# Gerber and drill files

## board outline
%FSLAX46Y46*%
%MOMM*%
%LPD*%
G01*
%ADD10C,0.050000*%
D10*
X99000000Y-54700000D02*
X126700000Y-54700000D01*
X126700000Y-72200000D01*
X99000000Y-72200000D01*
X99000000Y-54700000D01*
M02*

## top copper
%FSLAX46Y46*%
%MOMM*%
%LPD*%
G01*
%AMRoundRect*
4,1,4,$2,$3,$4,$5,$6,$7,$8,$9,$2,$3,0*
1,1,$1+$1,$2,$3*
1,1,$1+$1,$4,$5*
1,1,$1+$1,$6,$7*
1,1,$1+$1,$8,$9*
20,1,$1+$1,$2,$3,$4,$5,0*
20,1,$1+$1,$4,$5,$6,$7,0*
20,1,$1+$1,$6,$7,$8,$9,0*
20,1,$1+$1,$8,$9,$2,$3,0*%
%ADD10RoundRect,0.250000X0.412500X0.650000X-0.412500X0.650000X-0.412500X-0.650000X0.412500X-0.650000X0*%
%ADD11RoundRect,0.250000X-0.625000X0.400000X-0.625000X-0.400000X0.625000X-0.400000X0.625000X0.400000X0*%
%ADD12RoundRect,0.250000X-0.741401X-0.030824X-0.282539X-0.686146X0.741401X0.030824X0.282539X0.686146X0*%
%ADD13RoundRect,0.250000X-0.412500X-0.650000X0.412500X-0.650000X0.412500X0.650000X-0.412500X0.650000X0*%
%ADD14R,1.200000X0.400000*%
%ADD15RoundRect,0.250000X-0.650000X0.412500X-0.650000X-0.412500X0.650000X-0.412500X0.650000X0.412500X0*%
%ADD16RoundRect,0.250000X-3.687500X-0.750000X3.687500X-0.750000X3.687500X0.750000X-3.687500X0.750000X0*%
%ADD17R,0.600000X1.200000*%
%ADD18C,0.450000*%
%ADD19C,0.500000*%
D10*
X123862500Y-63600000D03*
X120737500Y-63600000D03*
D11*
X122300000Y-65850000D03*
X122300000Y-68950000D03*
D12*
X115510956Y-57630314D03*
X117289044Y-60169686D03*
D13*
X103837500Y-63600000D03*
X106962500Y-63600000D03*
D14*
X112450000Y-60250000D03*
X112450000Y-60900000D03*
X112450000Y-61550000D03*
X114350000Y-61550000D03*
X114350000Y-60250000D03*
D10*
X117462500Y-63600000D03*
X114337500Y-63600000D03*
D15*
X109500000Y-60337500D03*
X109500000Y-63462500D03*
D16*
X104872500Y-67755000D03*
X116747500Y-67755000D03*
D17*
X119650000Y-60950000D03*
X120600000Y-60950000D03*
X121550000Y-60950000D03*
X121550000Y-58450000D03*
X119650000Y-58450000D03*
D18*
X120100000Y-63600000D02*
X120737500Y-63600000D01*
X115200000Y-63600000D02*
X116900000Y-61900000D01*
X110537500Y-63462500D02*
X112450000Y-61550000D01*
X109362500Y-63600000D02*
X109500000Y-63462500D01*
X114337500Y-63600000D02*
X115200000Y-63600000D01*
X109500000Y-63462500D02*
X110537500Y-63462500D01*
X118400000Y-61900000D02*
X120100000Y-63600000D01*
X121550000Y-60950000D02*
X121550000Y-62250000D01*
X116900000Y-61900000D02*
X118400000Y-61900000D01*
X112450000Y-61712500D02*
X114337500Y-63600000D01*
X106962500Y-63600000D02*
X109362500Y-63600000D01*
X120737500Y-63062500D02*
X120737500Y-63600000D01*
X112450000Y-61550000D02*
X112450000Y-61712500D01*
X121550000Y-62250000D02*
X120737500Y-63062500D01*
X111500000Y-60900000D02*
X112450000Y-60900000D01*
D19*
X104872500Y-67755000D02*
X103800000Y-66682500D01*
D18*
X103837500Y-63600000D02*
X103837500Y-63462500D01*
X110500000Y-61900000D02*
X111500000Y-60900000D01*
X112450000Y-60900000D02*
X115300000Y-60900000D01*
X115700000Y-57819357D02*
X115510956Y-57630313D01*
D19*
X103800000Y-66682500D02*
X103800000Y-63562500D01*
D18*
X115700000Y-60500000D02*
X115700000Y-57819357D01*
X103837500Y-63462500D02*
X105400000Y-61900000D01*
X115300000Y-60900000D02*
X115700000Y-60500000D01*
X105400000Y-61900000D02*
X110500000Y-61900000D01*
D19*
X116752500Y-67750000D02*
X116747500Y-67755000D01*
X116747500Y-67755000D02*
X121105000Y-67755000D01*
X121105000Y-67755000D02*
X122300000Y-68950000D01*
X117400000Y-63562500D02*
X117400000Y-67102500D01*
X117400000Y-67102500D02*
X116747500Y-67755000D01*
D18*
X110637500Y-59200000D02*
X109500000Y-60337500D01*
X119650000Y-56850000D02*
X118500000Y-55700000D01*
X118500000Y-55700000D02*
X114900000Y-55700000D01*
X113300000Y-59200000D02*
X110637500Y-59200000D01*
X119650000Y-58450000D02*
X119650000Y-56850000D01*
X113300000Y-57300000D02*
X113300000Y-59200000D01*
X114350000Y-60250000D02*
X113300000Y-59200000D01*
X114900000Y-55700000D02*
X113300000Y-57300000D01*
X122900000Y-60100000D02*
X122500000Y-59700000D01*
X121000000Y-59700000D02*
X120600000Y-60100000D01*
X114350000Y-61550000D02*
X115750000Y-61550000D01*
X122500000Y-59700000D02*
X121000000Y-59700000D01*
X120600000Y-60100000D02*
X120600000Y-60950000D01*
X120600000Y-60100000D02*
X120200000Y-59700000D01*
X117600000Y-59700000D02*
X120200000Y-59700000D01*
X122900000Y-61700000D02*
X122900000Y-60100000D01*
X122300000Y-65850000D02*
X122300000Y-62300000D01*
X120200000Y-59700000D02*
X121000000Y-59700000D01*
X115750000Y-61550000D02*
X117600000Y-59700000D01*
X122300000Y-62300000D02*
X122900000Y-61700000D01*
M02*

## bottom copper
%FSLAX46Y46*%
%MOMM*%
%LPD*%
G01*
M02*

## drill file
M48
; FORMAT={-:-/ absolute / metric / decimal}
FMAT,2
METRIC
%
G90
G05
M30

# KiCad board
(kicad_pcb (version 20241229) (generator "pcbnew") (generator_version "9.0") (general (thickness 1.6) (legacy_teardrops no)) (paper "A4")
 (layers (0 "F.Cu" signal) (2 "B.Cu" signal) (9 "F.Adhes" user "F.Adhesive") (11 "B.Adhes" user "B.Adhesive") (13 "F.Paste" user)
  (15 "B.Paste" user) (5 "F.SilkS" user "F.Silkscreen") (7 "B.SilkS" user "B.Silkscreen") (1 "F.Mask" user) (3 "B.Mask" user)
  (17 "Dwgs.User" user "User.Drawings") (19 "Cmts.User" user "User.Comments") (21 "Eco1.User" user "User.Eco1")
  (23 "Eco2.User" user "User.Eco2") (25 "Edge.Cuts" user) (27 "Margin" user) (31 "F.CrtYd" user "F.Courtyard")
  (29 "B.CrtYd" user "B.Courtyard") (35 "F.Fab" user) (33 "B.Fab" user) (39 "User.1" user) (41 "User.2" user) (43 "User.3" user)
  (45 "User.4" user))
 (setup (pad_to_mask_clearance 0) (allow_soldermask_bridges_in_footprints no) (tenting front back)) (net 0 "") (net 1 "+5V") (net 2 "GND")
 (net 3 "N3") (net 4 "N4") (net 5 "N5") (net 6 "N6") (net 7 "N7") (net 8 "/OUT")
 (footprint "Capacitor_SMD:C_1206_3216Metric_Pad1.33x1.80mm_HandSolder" (layer "F.Cu") (at 122.3 63.6 180)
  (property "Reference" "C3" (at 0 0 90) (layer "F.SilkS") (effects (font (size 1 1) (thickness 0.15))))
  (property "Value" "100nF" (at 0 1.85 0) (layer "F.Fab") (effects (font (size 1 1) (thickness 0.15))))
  (pad "1" smd roundrect (at -1.5625 0 180) (size 1.325 1.8) (layers "F.Cu" "F.Mask" "F.Paste") (roundrect_rratio 0.188679) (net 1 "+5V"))
  (pad "2" smd roundrect (at 1.5625 0 180) (size 1.325 1.8) (layers "F.Cu" "F.Mask" "F.Paste") (roundrect_rratio 0.188679) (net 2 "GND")))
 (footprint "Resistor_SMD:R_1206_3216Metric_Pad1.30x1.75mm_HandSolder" (layer "F.Cu") (at 122.3 67.4 -90)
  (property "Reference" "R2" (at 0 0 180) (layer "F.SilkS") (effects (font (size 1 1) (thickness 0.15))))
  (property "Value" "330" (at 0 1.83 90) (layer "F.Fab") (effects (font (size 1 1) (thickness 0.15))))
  (pad "1" smd roundrect (at -1.55 0 270) (size 1.3 1.75) (layers "F.Cu" "F.Mask" "F.Paste") (roundrect_rratio 0.192308) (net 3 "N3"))
  (pad "2" smd roundrect (at 1.55 0 270) (size 1.3 1.75) (layers "F.Cu" "F.Mask" "F.Paste") (roundrect_rratio 0.192308) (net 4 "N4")))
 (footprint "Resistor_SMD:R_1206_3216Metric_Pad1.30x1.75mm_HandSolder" (layer "F.Cu") (at 116.4 58.9 -55)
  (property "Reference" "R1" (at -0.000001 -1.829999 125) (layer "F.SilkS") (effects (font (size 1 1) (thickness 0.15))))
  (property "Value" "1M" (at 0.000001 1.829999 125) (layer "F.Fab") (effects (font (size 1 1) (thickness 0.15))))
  (pad "1" smd roundrect (at -1.550001 0 305) (size 1.3 1.75) (layers "F.Cu" "F.Mask" "F.Paste") (roundrect_rratio 0.192308) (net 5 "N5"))
  (pad "2" smd roundrect (at 1.550001 0 305) (size 1.3 1.75) (layers "F.Cu" "F.Mask" "F.Paste") (roundrect_rratio 0.192308) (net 3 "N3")))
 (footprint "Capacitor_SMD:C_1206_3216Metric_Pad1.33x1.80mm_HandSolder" (layer "F.Cu") (at 105.4 63.6)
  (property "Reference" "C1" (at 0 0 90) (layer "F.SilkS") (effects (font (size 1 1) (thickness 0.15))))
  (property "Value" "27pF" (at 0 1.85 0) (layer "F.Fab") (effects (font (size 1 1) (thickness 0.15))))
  (pad "1" smd roundrect (at -1.5625 0) (size 1.325 1.8) (layers "F.Cu" "F.Mask" "F.Paste") (roundrect_rratio 0.188679) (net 5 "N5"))
  (pad "2" smd roundrect (at 1.5625 0) (size 1.325 1.8) (layers "F.Cu" "F.Mask" "F.Paste") (roundrect_rratio 0.188679) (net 2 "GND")))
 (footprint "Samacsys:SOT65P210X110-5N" (layer "F.Cu") (at 113.4 60.9)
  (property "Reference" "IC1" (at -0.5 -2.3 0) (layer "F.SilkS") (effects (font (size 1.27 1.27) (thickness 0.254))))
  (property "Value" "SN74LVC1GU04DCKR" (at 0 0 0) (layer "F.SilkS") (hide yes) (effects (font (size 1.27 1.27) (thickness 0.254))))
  (pad "1" smd rect (at -0.95 -0.65 90) (size 0.4 1.2) (layers "F.Cu" "F.Mask" "F.Paste") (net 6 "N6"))
  (pad "2" smd rect (at -0.95 0 90) (size 0.4 1.2) (layers "F.Cu" "F.Mask" "F.Paste") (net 5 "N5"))
  (pad "3" smd rect (at -0.95 0.65 90) (size 0.4 1.2) (layers "F.Cu" "F.Mask" "F.Paste") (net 2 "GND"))
  (pad "4" smd rect (at 0.95 0.65 90) (size 0.4 1.2) (layers "F.Cu" "F.Mask" "F.Paste") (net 3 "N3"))
  (pad "5" smd rect (at 0.95 -0.65 90) (size 0.4 1.2) (layers "F.Cu" "F.Mask" "F.Paste") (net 1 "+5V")))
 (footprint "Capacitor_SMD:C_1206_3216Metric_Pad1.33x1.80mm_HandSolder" (layer "F.Cu") (at 115.9 63.6 180)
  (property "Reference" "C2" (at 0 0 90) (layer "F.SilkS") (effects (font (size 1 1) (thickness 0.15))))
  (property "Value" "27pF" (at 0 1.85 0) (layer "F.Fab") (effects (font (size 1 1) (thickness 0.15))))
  (pad "1" smd roundrect (at -1.5625 0 180) (size 1.325 1.8) (layers "F.Cu" "F.Mask" "F.Paste") (roundrect_rratio 0.188679) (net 4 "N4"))
  (pad "2" smd roundrect (at 1.5625 0 180) (size 1.325 1.8) (layers "F.Cu" "F.Mask" "F.Paste") (roundrect_rratio 0.188679) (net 2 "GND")))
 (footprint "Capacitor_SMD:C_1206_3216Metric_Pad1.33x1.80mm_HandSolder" (layer "F.Cu") (at 109.5 61.9 -90)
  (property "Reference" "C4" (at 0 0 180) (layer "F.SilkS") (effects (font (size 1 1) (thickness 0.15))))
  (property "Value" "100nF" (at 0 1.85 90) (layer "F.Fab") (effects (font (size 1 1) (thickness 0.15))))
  (pad "1" smd roundrect (at -1.5625 0 270) (size 1.325 1.8) (layers "F.Cu" "F.Mask" "F.Paste") (roundrect_rratio 0.188679) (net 1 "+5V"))
  (pad "2" smd roundrect (at 1.5625 0 270) (size 1.325 1.8) (layers "F.Cu" "F.Mask" "F.Paste") (roundrect_rratio 0.188679) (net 2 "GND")))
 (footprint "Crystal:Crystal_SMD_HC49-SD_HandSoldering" (layer "F.Cu") (at 110.81 67.755)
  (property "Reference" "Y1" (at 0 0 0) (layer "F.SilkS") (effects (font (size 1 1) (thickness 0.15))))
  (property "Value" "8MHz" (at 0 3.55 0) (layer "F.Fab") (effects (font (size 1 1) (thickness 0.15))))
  (pad "1" smd roundrect (at -5.9375 0) (size 7.875 2) (layers "F.Cu" "F.Mask" "F.Paste") (roundrect_rratio 0.125) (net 5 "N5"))
  (pad "2" smd roundrect (at 5.9375 0) (size 7.875 2) (layers "F.Cu" "F.Mask" "F.Paste") (roundrect_rratio 0.125) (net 4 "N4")))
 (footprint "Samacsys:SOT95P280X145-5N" (layer "F.Cu") (at 120.6 59.7 90)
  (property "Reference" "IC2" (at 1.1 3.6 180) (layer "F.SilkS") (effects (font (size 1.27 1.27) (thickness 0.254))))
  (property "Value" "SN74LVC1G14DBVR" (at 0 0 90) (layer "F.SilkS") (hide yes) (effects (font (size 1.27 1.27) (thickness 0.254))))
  (pad "1" smd rect (at -1.25 -0.95 180) (size 0.6 1.2) (layers "F.Cu" "F.Mask" "F.Paste") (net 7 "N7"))
  (pad "2" smd rect (at -1.25 0 180) (size 0.6 1.2) (layers "F.Cu" "F.Mask" "F.Paste") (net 3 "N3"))
  (pad "3" smd rect (at -1.25 0.95 180) (size 0.6 1.2) (layers "F.Cu" "F.Mask" "F.Paste") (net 2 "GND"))
  (pad "4" smd rect (at 1.25 0.95 180) (size 0.6 1.2) (layers "F.Cu" "F.Mask" "F.Paste") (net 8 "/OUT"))
  (pad "5" smd rect (at 1.25 -0.95 180) (size 0.6 1.2) (layers "F.Cu" "F.Mask" "F.Paste") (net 1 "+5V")))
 (gr_rect (start 99 54.7) (end 126.7 72.2) (stroke (width 0.05) (type default)) (fill no) (layer "Edge.Cuts"))
 (segment (start 120.1 63.6) (end 120.7375 63.6) (width 0.45) (layer "F.Cu") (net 2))
 (segment (start 115.2 63.6) (end 116.9 61.9) (width 0.45) (layer "F.Cu") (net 2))
 (segment (start 110.5375 63.4625) (end 112.45 61.55) (width 0.45) (layer "F.Cu") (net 2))
 (segment (start 109.3625 63.6) (end 109.5 63.4625) (width 0.45) (layer "F.Cu") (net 2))
 (segment (start 114.3375 63.6) (end 115.2 63.6) (width 0.45) (layer "F.Cu") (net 2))
 (segment (start 109.5 63.4625) (end 110.5375 63.4625) (width 0.45) (layer "F.Cu") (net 2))
 (segment (start 118.4 61.9) (end 120.1 63.6) (width 0.45) (layer "F.Cu") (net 2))
 (segment (start 121.55 60.95) (end 121.55 62.25) (width 0.45) (layer "F.Cu") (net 2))
 (segment (start 116.9 61.9) (end 118.4 61.9) (width 0.45) (layer "F.Cu") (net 2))
 (segment (start 112.45 61.7125) (end 114.3375 63.6) (width 0.45) (layer "F.Cu") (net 2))
 (segment (start 106.9625 63.6) (end 109.3625 63.6) (width 0.45) (layer "F.Cu") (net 2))
 (segment (start 120.7375 63.0625) (end 120.7375 63.6) (width 0.45) (layer "F.Cu") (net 2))
 (segment (start 112.45 61.55) (end 112.45 61.7125) (width 0.45) (layer "F.Cu") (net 2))
 (segment (start 121.55 62.25) (end 120.7375 63.0625) (width 0.45) (layer "F.Cu") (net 2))
 (segment (start 111.5 60.9) (end 112.45 60.9) (width 0.45) (layer "F.Cu") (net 5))
 (segment (start 104.8725 67.755) (end 103.8 66.6825) (width 0.5) (layer "F.Cu") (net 5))
 (segment (start 103.8375 63.6) (end 103.8375 63.4625) (width 0.45) (layer "F.Cu") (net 5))
 (segment (start 110.5 61.9) (end 111.5 60.9) (width 0.45) (layer "F.Cu") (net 5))
 (segment (start 112.45 60.9) (end 115.3 60.9) (width 0.45) (layer "F.Cu") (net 5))
 (segment (start 115.7 57.819357) (end 115.510956 57.630313) (width 0.45) (layer "F.Cu") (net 5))
 (segment (start 103.8 66.6825) (end 103.8 63.5625) (width 0.5) (layer "F.Cu") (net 5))
 (segment (start 115.7 60.5) (end 115.7 57.819357) (width 0.45) (layer "F.Cu") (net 5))
 (segment (start 103.8375 63.4625) (end 105.4 61.9) (width 0.45) (layer "F.Cu") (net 5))
 (segment (start 115.3 60.9) (end 115.7 60.5) (width 0.45) (layer "F.Cu") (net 5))
 (segment (start 105.4 61.9) (end 110.5 61.9) (width 0.45) (layer "F.Cu") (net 5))
 (segment (start 116.7525 67.75) (end 116.7475 67.755) (width 0.5) (layer "F.Cu") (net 4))
 (segment (start 116.7475 67.755) (end 121.105 67.755) (width 0.5) (layer "F.Cu") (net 4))
 (segment (start 121.105 67.755) (end 122.3 68.95) (width 0.5) (layer "F.Cu") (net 4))
 (segment (start 117.4 63.5625) (end 117.4 67.1025) (width 0.5) (layer "F.Cu") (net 4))
 (segment (start 117.4 67.1025) (end 116.7475 67.755) (width 0.5) (layer "F.Cu") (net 4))
 (segment (start 110.6375 59.2) (end 109.5 60.3375) (width 0.45) (layer "F.Cu") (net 1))
 (segment (start 119.65 56.85) (end 118.5 55.7) (width 0.45) (layer "F.Cu") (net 1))
 (segment (start 118.5 55.7) (end 114.9 55.7) (width 0.45) (layer "F.Cu") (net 1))
 (segment (start 113.3 59.2) (end 110.6375 59.2) (width 0.45) (layer "F.Cu") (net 1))
 (segment (start 119.65 58.45) (end 119.65 56.85) (width 0.45) (layer "F.Cu") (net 1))
 (segment (start 113.3 57.3) (end 113.3 59.2) (width 0.45) (layer "F.Cu") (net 1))
 (segment (start 114.35 60.25) (end 113.3 59.2) (width 0.45) (layer "F.Cu") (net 1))
 (segment (start 114.9 55.7) (end 113.3 57.3) (width 0.45) (layer "F.Cu") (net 1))
 (segment (start 122.9 60.1) (end 122.5 59.7) (width 0.45) (layer "F.Cu") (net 3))
 (segment (start 121 59.7) (end 120.6 60.1) (width 0.45) (layer "F.Cu") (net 3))
 (segment (start 114.35 61.55) (end 115.75 61.55) (width 0.45) (layer "F.Cu") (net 3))
 (segment (start 122.5 59.7) (end 121 59.7) (width 0.45) (layer "F.Cu") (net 3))
 (segment (start 120.6 60.1) (end 120.6 60.95) (width 0.45) (layer "F.Cu") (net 3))
 (segment (start 120.6 60.1) (end 120.2 59.7) (width 0.45) (layer "F.Cu") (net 3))
 (segment (start 117.6 59.7) (end 120.2 59.7) (width 0.45) (layer "F.Cu") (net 3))
 (segment (start 122.9 61.7) (end 122.9 60.1) (width 0.45) (layer "F.Cu") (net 3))
 (segment (start 122.3 65.85) (end 122.3 62.3) (width 0.45) (layer "F.Cu") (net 3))
 (segment (start 120.2 59.7) (end 121 59.7) (width 0.45) (layer "F.Cu") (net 3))
 (segment (start 115.75 61.55) (end 117.6 59.7) (width 0.45) (layer "F.Cu") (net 3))
 (segment (start 122.3 62.3) (end 122.9 61.7) (width 0.45) (layer "F.Cu") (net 3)))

